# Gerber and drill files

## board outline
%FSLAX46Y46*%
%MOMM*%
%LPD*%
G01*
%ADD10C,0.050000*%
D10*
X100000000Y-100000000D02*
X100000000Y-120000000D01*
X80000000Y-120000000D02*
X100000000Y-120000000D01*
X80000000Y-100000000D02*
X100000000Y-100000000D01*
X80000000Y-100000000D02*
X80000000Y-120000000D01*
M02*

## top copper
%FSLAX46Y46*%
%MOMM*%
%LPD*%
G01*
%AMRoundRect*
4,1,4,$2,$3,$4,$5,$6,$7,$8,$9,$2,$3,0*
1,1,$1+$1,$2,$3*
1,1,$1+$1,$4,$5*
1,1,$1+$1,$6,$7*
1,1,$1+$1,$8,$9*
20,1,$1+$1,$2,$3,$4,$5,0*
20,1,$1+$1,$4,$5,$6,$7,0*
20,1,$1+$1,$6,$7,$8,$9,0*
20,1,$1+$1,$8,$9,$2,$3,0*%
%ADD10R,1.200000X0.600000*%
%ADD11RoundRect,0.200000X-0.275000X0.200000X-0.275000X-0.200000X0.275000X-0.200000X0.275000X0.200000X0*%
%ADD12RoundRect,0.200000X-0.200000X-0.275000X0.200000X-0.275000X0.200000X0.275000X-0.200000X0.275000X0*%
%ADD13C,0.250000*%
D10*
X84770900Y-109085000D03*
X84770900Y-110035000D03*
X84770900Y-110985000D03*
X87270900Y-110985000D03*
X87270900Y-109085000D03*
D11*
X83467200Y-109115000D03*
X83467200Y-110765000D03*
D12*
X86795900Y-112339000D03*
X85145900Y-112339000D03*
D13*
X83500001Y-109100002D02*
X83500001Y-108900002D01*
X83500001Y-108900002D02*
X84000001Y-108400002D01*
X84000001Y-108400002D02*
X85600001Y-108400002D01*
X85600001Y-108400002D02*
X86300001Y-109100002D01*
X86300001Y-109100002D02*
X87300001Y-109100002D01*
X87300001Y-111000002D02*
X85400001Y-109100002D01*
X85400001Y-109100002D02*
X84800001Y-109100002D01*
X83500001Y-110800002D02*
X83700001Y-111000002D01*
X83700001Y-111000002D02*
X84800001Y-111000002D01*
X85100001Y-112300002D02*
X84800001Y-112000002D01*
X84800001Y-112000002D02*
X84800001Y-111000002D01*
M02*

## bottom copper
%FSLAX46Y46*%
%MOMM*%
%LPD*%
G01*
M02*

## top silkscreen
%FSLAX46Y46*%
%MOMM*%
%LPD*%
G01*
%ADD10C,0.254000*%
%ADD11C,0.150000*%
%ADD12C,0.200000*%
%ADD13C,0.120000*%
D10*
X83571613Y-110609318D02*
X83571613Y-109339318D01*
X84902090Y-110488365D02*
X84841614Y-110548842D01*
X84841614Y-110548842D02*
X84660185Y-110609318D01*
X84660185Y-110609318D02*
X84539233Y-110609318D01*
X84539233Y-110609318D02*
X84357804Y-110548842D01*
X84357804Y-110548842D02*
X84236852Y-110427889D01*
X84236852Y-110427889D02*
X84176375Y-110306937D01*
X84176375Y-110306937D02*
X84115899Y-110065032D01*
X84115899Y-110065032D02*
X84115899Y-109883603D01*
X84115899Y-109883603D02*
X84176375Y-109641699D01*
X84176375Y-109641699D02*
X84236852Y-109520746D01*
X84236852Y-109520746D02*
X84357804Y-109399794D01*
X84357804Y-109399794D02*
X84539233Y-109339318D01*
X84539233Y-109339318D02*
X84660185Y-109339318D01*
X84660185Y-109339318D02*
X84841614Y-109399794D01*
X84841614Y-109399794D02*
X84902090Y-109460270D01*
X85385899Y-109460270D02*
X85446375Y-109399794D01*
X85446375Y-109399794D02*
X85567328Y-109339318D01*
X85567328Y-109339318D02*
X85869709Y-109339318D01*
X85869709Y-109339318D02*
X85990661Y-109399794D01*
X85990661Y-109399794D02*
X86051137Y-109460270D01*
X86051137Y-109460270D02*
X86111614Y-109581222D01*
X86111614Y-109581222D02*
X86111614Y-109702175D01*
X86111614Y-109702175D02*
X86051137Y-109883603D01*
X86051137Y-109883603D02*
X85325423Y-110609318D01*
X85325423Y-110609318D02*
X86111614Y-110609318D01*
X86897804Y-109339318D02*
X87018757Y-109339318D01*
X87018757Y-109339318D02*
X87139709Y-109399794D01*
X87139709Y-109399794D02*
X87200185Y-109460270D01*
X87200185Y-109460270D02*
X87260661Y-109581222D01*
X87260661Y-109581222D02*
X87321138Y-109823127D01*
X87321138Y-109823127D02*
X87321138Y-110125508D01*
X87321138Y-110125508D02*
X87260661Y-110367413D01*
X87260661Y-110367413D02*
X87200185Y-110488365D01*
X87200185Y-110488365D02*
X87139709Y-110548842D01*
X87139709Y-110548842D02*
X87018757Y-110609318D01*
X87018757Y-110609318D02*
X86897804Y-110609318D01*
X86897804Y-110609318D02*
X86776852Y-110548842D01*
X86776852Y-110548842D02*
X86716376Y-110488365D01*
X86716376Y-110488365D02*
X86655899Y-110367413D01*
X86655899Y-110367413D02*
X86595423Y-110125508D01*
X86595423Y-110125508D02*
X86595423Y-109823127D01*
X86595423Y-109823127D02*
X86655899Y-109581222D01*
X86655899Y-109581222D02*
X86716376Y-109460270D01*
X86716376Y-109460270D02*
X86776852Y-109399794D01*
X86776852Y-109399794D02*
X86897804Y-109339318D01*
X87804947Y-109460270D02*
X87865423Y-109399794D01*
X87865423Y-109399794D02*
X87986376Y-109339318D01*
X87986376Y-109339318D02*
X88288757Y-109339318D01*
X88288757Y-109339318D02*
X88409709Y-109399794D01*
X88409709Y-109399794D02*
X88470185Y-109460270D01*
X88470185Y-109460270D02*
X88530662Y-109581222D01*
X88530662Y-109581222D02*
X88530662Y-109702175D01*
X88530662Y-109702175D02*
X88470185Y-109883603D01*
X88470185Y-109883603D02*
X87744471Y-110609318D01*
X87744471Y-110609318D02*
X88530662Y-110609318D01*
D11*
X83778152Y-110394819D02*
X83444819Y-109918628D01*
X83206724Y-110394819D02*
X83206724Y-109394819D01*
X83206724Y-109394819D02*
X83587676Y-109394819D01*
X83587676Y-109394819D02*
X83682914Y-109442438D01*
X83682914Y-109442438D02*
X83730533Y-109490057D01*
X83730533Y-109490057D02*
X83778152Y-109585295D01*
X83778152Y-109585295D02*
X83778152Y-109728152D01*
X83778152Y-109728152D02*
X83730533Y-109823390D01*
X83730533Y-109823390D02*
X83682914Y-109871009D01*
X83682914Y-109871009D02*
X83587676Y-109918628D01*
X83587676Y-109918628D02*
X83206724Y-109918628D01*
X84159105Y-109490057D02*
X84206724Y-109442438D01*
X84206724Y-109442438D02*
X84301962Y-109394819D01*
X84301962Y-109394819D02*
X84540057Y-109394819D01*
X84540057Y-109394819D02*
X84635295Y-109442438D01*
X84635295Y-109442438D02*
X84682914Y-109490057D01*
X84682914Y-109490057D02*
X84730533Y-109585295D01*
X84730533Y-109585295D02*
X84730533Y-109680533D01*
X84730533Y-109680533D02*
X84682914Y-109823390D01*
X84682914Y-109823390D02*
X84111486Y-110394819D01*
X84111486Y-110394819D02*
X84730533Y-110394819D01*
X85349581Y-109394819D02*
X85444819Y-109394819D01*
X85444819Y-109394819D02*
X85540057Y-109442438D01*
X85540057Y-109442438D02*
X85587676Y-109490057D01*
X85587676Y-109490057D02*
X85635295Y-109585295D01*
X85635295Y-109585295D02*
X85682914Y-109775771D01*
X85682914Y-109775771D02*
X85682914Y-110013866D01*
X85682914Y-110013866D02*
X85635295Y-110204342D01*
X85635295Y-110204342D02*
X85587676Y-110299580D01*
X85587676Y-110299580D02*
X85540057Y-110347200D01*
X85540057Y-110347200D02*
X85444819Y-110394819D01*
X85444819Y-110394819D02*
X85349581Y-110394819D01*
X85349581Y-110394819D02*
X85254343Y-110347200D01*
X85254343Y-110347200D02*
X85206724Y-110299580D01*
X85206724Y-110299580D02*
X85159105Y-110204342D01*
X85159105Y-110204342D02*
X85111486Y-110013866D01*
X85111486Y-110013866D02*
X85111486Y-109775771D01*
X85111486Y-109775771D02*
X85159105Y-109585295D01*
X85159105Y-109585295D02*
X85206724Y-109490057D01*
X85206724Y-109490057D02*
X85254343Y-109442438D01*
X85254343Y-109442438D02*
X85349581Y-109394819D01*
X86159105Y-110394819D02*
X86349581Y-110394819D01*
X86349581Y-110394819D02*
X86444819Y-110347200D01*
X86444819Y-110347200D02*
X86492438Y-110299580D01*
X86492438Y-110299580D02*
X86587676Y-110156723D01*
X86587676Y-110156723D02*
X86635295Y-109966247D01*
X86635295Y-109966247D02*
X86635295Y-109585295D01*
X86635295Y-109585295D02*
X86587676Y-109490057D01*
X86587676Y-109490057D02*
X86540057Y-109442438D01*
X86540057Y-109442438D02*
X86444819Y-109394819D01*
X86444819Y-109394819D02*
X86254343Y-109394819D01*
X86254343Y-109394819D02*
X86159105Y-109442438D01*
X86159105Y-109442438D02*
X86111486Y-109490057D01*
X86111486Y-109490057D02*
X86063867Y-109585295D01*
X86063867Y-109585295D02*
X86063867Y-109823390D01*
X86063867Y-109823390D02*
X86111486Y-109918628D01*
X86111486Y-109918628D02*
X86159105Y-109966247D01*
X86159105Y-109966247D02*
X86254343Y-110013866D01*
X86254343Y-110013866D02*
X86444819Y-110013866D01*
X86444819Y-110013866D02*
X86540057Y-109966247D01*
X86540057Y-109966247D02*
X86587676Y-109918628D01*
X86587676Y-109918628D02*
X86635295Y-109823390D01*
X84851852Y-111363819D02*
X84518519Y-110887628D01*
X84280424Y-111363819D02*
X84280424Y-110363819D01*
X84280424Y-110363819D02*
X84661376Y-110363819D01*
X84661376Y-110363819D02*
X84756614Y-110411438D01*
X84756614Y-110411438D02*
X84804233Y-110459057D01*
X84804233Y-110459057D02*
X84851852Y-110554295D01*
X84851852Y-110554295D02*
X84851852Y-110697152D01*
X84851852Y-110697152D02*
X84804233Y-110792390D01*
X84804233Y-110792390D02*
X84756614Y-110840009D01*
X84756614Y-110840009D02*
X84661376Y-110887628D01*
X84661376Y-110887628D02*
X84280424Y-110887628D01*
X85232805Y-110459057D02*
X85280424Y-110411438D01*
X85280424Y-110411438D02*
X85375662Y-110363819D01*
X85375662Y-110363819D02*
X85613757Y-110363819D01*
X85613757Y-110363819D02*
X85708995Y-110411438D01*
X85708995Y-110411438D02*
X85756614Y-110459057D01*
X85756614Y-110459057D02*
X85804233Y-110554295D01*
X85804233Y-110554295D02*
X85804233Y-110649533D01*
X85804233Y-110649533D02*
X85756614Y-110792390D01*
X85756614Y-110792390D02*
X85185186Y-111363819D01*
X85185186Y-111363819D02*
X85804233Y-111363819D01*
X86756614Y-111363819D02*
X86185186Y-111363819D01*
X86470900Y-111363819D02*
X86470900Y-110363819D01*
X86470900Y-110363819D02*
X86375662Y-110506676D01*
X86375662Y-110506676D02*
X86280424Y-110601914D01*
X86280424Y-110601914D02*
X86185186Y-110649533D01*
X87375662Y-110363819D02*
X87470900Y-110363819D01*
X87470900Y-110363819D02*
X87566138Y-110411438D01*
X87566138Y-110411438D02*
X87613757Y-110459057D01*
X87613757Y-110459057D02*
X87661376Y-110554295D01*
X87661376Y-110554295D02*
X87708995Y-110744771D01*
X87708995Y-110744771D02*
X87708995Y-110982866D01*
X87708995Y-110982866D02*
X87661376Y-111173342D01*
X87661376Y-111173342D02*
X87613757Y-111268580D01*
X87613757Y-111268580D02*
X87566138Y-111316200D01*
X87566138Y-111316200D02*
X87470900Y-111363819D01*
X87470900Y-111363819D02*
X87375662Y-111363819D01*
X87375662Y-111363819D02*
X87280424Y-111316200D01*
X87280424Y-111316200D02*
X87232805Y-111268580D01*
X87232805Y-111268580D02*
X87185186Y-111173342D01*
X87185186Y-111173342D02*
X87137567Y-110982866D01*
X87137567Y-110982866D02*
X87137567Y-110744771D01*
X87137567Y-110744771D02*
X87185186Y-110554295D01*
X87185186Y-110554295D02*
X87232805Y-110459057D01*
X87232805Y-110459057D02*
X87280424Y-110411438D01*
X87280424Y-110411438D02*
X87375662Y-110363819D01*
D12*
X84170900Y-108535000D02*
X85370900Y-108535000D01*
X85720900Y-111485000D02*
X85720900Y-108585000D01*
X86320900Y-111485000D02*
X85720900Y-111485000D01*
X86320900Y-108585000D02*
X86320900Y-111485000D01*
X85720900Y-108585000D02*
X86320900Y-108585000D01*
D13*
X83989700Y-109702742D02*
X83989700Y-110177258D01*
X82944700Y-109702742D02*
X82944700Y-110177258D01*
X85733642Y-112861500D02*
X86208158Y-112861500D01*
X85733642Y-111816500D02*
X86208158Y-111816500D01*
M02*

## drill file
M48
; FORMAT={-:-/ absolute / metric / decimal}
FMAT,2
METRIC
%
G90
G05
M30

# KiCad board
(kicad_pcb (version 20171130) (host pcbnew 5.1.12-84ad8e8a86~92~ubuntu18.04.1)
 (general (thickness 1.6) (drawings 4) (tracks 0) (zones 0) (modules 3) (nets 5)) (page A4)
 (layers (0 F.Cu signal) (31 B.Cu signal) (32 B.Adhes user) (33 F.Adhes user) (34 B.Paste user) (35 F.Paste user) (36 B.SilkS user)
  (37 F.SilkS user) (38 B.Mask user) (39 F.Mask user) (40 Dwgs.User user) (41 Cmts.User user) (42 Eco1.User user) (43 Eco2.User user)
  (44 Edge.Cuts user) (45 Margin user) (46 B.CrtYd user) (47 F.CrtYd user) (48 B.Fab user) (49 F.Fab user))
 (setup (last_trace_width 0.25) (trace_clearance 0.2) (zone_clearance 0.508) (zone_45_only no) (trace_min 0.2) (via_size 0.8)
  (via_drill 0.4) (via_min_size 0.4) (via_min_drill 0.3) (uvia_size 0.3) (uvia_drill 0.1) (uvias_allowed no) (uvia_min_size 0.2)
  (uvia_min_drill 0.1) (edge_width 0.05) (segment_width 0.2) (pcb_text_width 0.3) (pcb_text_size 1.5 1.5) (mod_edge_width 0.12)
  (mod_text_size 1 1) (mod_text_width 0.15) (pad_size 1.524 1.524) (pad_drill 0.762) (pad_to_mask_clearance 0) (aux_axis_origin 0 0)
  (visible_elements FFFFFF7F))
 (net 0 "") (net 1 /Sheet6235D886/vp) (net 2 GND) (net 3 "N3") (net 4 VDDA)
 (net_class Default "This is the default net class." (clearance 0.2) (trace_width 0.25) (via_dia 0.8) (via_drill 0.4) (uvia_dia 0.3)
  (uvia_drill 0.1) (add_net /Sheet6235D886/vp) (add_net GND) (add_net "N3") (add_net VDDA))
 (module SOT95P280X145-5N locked (layer F.Cu) (at 86.020900 110.035000)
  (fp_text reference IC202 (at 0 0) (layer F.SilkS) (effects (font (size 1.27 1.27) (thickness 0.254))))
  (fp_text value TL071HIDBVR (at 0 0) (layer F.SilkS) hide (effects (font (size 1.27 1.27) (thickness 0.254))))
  (fp_line (start -1.85 -1.5) (end -0.65 -1.5) (layer F.SilkS) (width 0.2))
  (fp_line (start -0.3 1.45) (end -0.3 -1.45) (layer F.SilkS) (width 0.2))
  (fp_line (start 0.3 1.45) (end -0.3 1.45) (layer F.SilkS) (width 0.2))
  (fp_line (start 0.3 -1.45) (end 0.3 1.45) (layer F.SilkS) (width 0.2))
  (fp_line (start -0.3 -1.45) (end 0.3 -1.45) (layer F.SilkS) (width 0.2))
  (pad 1 smd rect (at -1.25 -0.95 90.000000) (size 0.6 1.2) (layers F.Cu F.Mask F.Paste) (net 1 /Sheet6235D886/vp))
  (pad 2 smd rect (at -1.25 0 90.000000) (size 0.6 1.2) (layers F.Cu F.Mask F.Paste) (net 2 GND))
  (pad 3 smd rect (at -1.25 0.95 90.000000) (size 0.6 1.2) (layers F.Cu F.Mask F.Paste) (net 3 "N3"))
  (pad 4 smd rect (at 1.25 0.95 90.000000) (size 0.6 1.2) (layers F.Cu F.Mask F.Paste) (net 1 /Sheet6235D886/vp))
  (pad 5 smd rect (at 1.25 -0.95 90.000000) (size 0.6 1.2) (layers F.Cu F.Mask F.Paste) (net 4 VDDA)))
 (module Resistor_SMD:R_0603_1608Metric (layer F.Cu) (at 83.467200 109.940000 270.000000)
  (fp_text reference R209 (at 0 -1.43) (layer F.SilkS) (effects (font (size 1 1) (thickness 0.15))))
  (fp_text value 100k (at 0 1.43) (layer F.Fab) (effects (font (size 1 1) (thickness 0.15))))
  (fp_line (start -0.237258 -0.5225) (end 0.237258 -0.5225) (layer F.SilkS) (width 0.12))
  (fp_line (start -0.237258 0.5225) (end 0.237258 0.5225) (layer F.SilkS) (width 0.12))
  (pad 1 smd roundrect (at -0.825 0 270.000000) (size 0.8 0.95) (layers F.Cu F.Mask F.Paste) (roundrect_rratio 0.25) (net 4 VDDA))
  (pad 2 smd roundrect (at 0.825 0 270.000000) (size 0.8 0.95) (layers F.Cu F.Mask F.Paste) (roundrect_rratio 0.25) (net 3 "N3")))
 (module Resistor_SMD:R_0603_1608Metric (layer F.Cu) (at 85.970900 112.339000)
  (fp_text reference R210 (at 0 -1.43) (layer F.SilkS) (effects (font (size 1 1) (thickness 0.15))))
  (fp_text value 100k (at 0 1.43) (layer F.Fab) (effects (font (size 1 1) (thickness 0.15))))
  (fp_line (start -0.237258 0.5225) (end 0.237258 0.5225) (layer F.SilkS) (width 0.12))
  (fp_line (start -0.237258 -0.5225) (end 0.237258 -0.5225) (layer F.SilkS) (width 0.12))
  (pad 2 smd roundrect (at 0.825 0) (size 0.8 0.95) (layers F.Cu F.Mask F.Paste) (roundrect_rratio 0.25) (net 2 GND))
  (pad 1 smd roundrect (at -0.825 0) (size 0.8 0.95) (layers F.Cu F.Mask F.Paste) (roundrect_rratio 0.25) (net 3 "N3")))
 (gr_line (start 100 100) (end 100 120) (layer Edge.Cuts) (width 0.05))
 (gr_line (start 80 120) (end 100 120) (layer Edge.Cuts) (width 0.05))
 (gr_line (start 80 100) (end 100 100) (layer Edge.Cuts) (width 0.05))
 (gr_line (start 80 100) (end 80 120) (layer Edge.Cuts) (width 0.05))
 (segment (start 83.500001 109.100002) (end 83.500001 108.900002) (width 0.250000) (layer F.Cu) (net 4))
 (segment (start 83.500001 108.900002) (end 84.000001 108.400002) (width 0.250000) (layer F.Cu) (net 4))
 (segment (start 84.000001 108.400002) (end 85.600001 108.400002) (width 0.250000) (layer F.Cu) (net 4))
 (segment (start 85.600001 108.400002) (end 86.300001 109.100002) (width 0.250000) (layer F.Cu) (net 4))
 (segment (start 86.300001 109.100002) (end 87.300001 109.100002) (width 0.250000) (layer F.Cu) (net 4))
 (segment (start 87.300001 111.000002) (end 85.400001 109.100002) (width 0.250000) (layer F.Cu) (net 1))
 (segment (start 85.400001 109.100002) (end 84.800001 109.100002) (width 0.250000) (layer F.Cu) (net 1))
 (segment (start 83.500001 110.800002) (end 83.700001 111.000002) (width 0.250000) (layer F.Cu) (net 3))
 (segment (start 83.700001 111.000002) (end 84.800001 111.000002) (width 0.250000) (layer F.Cu) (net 3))
 (segment (start 85.100001 112.300002) (end 84.800001 112.000002) (width 0.250000) (layer F.Cu) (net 3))
 (segment (start 84.800001 112.000002) (end 84.800001 111.000002) (width 0.250000) (layer F.Cu) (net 3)))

